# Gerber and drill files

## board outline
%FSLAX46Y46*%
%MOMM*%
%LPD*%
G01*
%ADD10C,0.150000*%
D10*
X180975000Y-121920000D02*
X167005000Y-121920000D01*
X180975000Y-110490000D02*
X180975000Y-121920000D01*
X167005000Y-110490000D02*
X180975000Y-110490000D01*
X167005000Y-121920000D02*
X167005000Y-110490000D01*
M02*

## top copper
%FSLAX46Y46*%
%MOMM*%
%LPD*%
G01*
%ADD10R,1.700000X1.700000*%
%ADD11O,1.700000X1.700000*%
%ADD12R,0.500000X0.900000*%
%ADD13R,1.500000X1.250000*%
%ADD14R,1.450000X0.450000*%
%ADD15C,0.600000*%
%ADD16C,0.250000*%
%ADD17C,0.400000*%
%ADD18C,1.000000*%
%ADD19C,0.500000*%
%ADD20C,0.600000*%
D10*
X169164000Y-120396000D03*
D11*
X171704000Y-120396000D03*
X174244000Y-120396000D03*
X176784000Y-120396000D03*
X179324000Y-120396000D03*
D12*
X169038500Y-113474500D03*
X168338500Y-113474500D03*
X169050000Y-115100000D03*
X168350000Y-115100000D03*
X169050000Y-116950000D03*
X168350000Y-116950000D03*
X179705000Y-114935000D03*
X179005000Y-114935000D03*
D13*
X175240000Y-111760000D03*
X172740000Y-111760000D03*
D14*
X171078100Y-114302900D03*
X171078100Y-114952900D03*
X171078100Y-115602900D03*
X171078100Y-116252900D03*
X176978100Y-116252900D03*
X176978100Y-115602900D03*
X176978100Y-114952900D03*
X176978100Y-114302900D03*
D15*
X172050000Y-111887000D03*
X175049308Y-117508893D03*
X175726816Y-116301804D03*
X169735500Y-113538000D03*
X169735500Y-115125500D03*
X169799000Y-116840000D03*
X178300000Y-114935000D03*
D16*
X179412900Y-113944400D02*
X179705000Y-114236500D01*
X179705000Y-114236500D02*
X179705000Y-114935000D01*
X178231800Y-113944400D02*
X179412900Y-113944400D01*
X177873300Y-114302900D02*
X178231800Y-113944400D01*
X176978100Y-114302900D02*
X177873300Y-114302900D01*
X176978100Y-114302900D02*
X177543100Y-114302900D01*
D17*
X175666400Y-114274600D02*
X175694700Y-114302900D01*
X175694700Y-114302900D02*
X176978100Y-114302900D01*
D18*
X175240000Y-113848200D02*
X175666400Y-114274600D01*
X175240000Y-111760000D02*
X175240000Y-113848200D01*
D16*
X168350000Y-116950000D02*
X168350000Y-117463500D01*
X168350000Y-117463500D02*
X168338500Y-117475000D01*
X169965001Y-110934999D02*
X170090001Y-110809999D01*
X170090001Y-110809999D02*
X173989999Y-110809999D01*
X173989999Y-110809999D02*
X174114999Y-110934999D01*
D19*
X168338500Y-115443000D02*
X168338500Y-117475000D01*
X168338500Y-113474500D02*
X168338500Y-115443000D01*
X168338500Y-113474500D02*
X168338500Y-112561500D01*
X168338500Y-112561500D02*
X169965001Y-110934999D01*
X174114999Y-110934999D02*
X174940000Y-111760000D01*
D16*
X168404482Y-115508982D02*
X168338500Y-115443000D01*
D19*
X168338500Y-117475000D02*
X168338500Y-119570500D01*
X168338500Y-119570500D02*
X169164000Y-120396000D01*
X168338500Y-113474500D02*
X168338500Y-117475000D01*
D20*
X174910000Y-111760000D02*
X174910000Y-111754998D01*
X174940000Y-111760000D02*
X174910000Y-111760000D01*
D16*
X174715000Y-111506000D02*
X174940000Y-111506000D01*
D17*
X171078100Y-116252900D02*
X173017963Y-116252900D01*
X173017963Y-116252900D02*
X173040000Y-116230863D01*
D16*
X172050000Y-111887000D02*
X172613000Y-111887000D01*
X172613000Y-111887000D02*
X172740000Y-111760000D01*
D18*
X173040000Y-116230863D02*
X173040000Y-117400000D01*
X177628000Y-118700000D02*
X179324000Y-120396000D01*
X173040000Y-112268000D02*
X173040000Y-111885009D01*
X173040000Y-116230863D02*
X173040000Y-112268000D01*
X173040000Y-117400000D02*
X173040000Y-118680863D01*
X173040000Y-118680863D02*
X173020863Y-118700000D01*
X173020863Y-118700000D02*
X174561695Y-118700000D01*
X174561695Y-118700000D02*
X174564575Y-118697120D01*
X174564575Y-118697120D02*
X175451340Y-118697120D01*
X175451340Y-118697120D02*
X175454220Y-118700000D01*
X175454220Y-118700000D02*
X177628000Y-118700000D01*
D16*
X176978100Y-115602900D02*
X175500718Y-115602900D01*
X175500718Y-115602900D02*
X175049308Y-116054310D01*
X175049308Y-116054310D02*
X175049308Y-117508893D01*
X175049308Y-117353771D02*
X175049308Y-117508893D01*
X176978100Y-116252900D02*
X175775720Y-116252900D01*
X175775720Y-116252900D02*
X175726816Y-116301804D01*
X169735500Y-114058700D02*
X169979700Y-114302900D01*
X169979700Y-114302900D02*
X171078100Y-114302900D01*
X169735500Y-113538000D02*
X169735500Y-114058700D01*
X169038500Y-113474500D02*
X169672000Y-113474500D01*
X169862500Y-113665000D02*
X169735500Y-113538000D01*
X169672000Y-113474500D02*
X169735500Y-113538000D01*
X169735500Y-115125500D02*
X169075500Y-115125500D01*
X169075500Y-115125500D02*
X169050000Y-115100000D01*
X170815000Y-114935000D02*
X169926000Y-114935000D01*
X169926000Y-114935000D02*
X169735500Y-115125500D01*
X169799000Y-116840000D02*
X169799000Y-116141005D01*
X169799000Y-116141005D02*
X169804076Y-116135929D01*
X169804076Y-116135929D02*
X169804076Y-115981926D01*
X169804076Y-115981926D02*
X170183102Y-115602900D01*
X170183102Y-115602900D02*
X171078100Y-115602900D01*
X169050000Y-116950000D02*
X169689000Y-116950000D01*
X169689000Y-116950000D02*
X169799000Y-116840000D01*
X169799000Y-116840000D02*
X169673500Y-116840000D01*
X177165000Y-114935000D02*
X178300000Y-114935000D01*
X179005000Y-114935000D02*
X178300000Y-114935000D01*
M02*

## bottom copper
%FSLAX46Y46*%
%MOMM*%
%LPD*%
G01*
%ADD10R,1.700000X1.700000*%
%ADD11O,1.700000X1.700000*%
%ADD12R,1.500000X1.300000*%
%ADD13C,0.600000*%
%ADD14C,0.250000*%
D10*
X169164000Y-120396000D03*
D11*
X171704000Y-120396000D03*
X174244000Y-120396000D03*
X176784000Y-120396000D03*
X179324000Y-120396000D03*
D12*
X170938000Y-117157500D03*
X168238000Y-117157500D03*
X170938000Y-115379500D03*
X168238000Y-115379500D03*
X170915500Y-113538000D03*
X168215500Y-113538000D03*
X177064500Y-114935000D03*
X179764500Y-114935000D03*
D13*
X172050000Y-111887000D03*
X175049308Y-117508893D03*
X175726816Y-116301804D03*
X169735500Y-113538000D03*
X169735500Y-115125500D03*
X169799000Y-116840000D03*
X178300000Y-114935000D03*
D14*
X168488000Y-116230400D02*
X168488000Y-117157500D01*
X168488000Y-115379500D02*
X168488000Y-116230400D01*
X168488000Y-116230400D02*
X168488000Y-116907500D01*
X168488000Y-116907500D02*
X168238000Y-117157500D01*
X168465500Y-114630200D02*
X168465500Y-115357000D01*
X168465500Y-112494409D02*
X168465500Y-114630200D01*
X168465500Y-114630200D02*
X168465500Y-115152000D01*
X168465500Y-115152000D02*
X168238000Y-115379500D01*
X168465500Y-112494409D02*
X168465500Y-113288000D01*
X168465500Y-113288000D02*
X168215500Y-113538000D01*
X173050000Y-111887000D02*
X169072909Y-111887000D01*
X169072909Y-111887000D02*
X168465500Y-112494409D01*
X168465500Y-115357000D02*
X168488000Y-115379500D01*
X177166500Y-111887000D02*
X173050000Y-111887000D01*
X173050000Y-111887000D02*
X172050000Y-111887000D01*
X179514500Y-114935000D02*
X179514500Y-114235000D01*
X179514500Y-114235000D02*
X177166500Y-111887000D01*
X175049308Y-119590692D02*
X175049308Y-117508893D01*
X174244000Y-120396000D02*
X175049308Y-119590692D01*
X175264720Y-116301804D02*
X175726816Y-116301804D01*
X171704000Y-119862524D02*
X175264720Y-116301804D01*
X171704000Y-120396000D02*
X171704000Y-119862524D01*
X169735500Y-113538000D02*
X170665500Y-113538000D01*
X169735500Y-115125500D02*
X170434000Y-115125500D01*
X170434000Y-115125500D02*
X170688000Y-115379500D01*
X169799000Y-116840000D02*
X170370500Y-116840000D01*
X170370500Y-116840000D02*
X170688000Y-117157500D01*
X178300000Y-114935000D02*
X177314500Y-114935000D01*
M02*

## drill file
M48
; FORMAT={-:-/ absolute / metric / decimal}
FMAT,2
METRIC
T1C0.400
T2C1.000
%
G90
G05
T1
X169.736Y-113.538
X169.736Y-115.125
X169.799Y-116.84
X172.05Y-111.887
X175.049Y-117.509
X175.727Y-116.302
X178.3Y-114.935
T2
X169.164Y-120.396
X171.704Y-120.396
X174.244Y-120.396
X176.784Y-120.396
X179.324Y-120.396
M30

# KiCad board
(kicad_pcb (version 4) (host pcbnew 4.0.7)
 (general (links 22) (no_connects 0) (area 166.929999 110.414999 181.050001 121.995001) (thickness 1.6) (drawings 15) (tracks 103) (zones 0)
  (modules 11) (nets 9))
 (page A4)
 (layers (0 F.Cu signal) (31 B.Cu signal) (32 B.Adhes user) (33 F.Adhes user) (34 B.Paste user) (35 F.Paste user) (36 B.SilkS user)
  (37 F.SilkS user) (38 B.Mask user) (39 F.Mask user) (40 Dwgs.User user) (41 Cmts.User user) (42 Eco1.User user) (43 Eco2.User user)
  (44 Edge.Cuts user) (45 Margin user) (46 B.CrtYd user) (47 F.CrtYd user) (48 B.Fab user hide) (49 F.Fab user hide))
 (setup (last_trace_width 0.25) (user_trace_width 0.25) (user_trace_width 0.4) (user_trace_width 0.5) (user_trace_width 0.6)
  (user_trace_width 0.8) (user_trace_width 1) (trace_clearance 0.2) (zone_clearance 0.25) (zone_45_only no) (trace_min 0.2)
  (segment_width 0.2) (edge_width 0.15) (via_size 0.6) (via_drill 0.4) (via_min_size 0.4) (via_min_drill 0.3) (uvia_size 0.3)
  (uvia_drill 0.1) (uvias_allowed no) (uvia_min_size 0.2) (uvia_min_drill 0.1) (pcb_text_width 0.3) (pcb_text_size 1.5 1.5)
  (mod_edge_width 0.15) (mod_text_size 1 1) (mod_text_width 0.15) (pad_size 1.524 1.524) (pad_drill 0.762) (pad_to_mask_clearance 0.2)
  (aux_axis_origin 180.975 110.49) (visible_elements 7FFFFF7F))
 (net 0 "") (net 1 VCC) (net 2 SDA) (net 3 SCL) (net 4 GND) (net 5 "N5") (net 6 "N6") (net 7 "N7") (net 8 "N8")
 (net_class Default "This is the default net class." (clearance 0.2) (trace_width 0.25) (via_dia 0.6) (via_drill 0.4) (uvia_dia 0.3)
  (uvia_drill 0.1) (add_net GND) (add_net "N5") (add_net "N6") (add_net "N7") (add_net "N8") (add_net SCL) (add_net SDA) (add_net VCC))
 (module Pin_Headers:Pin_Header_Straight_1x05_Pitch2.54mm (layer F.Cu) (at 169.164 120.396 90)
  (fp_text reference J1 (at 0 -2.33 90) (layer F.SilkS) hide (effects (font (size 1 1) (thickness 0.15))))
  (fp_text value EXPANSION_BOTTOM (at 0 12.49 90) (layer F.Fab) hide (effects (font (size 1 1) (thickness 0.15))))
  (pad 1 thru_hole rect (at 0 0 90) (size 1.7 1.7) (drill 1) (layers *.Cu *.Mask) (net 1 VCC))
  (pad 2 thru_hole oval (at 0 2.54 90) (size 1.7 1.7) (drill 1) (layers *.Cu *.Mask) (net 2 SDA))
  (pad 3 thru_hole oval (at 0 5.08 90) (size 1.7 1.7) (drill 1) (layers *.Cu *.Mask) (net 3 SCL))
  (pad 4 thru_hole oval (at 0 7.62 90) (size 1.7 1.7) (drill 1) (layers *.Cu *.Mask))
  (pad 5 thru_hole oval (at 0 10.16 90) (size 1.7 1.7) (drill 1) (layers *.Cu *.Mask) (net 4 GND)))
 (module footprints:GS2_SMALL (layer F.Cu) (at 168.3385 113.4745 270)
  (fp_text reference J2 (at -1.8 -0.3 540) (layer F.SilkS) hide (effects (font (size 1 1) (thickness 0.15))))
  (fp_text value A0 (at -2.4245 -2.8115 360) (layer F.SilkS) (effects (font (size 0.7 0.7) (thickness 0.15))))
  (pad 1 smd rect (at 0 -0.7 270) (size 0.9 0.5) (layers F.Cu F.Paste F.Mask) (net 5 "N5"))
  (pad 2 smd rect (at 0 0 270) (size 0.9 0.5) (layers F.Cu F.Paste F.Mask) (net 1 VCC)))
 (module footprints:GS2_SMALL (layer F.Cu) (at 168.35 115.1 270)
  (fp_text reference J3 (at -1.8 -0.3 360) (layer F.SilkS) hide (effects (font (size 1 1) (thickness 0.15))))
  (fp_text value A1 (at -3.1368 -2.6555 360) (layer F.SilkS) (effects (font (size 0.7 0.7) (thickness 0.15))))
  (pad 1 smd rect (at 0 -0.7 270) (size 0.9 0.5) (layers F.Cu F.Paste F.Mask) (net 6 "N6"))
  (pad 2 smd rect (at 0 0 270) (size 0.9 0.5) (layers F.Cu F.Paste F.Mask) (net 1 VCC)))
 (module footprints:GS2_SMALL (layer F.Cu) (at 168.35 116.95 270)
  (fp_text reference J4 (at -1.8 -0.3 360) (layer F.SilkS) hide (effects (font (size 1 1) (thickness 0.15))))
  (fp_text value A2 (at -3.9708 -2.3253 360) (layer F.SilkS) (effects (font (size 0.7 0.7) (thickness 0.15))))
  (pad 1 smd rect (at 0 -0.7 270) (size 0.9 0.5) (layers F.Cu F.Paste F.Mask) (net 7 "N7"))
  (pad 2 smd rect (at 0 0 270) (size 0.9 0.5) (layers F.Cu F.Paste F.Mask) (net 1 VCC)))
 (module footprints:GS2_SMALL (layer F.Cu) (at 179.005 114.935 270)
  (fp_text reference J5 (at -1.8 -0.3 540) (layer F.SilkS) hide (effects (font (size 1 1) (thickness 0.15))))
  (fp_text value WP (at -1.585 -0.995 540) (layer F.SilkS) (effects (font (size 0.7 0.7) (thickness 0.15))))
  (pad 1 smd rect (at 0 -0.7 270) (size 0.9 0.5) (layers F.Cu F.Paste F.Mask) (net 1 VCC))
  (pad 2 smd rect (at 0 0 270) (size 0.9 0.5) (layers F.Cu F.Paste F.Mask) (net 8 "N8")))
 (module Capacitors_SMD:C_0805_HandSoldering (layer F.Cu) (at 173.99 111.76 180)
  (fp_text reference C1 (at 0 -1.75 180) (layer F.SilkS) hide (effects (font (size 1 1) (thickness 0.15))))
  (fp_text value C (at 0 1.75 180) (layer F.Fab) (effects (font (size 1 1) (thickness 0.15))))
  (pad 1 smd rect (at -1.25 0 180) (size 1.5 1.25) (layers F.Cu F.Paste F.Mask) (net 1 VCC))
  (pad 2 smd rect (at 1.25 0 180) (size 1.5 1.25) (layers F.Cu F.Paste F.Mask) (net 4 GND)))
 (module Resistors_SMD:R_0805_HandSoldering (layer B.Cu) (at 169.588 117.1575 180)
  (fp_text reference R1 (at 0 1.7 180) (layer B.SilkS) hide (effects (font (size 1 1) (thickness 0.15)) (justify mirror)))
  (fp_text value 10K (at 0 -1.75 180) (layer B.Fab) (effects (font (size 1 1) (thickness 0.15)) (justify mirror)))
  (pad 1 smd rect (at -1.35 0 180) (size 1.5 1.3) (layers B.Cu B.Paste B.Mask) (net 7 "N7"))
  (pad 2 smd rect (at 1.35 0 180) (size 1.5 1.3) (layers B.Cu B.Paste B.Mask) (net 4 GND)))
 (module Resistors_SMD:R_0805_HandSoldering (layer B.Cu) (at 169.588 115.3795 180)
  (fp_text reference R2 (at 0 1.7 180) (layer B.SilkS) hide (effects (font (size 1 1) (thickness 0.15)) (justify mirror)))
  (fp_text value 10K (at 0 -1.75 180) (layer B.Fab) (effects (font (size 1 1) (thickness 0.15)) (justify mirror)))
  (pad 1 smd rect (at -1.35 0 180) (size 1.5 1.3) (layers B.Cu B.Paste B.Mask) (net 6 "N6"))
  (pad 2 smd rect (at 1.35 0 180) (size 1.5 1.3) (layers B.Cu B.Paste B.Mask) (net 4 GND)))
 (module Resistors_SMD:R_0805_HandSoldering (layer B.Cu) (at 169.5655 113.538 180)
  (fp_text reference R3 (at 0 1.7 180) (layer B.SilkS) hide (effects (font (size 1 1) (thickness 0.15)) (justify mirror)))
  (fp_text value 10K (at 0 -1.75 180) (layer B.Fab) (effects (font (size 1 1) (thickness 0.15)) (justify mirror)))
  (pad 1 smd rect (at -1.35 0 180) (size 1.5 1.3) (layers B.Cu B.Paste B.Mask) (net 5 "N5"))
  (pad 2 smd rect (at 1.35 0 180) (size 1.5 1.3) (layers B.Cu B.Paste B.Mask) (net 4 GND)))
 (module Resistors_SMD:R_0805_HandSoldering (layer B.Cu) (at 178.4145 114.935)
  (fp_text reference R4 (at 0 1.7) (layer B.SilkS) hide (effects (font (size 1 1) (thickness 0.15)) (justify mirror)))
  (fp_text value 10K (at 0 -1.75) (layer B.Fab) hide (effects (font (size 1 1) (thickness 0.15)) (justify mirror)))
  (pad 1 smd rect (at -1.35 0) (size 1.5 1.3) (layers B.Cu B.Paste B.Mask) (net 8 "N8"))
  (pad 2 smd rect (at 1.35 0) (size 1.5 1.3) (layers B.Cu B.Paste B.Mask) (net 4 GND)))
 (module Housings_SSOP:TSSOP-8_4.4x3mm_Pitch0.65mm (layer F.Cu) (at 174.0281 115.2779)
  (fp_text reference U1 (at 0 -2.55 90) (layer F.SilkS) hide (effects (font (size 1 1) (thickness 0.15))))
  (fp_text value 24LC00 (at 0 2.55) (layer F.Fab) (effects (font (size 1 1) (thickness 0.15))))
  (pad 1 smd rect (at -2.95 -0.975) (size 1.45 0.45) (layers F.Cu F.Paste F.Mask) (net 5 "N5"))
  (pad 2 smd rect (at -2.95 -0.325) (size 1.45 0.45) (layers F.Cu F.Paste F.Mask) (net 6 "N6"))
  (pad 3 smd rect (at -2.95 0.325) (size 1.45 0.45) (layers F.Cu F.Paste F.Mask) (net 7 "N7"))
  (pad 4 smd rect (at -2.95 0.975) (size 1.45 0.45) (layers F.Cu F.Paste F.Mask) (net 4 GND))
  (pad 5 smd rect (at 2.95 0.975) (size 1.45 0.45) (layers F.Cu F.Paste F.Mask) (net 2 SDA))
  (pad 6 smd rect (at 2.95 0.325) (size 1.45 0.45) (layers F.Cu F.Paste F.Mask) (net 3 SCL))
  (pad 7 smd rect (at 2.95 -0.325) (size 1.45 0.45) (layers F.Cu F.Paste F.Mask) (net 8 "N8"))
  (pad 8 smd rect (at 2.95 -0.975) (size 1.45 0.45) (layers F.Cu F.Paste F.Mask) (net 1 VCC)))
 (gr_line (start 180.975 121.92) (end 167.005 121.92) (layer Edge.Cuts) (width 0.15))
 (gr_line (start 180.975 110.49) (end 180.975 121.92) (layer Edge.Cuts) (width 0.15))
 (gr_line (start 167.005 110.49) (end 180.975 110.49) (layer Edge.Cuts) (width 0.15))
 (gr_line (start 167.005 121.92) (end 167.005 110.49) (layer Edge.Cuts) (width 0.15))
 (segment (start 179.4129 113.9444) (end 179.705 114.2365) (width 0.25) (layer F.Cu) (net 1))
 (segment (start 179.705 114.2365) (end 179.705 114.935) (width 0.25) (layer F.Cu) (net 1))
 (segment (start 178.2318 113.9444) (end 179.4129 113.9444) (width 0.25) (layer F.Cu) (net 1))
 (segment (start 177.8733 114.3029) (end 178.2318 113.9444) (width 0.25) (layer F.Cu) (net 1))
 (segment (start 176.9781 114.3029) (end 177.8733 114.3029) (width 0.25) (layer F.Cu) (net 1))
 (segment (start 176.9781 114.3029) (end 177.5431 114.3029) (width 0.25) (layer F.Cu) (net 1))
 (segment (start 175.6664 114.2746) (end 175.6947 114.3029) (width 0.4) (layer F.Cu) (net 1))
 (segment (start 175.6947 114.3029) (end 176.9781 114.3029) (width 0.4) (layer F.Cu) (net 1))
 (segment (start 175.24 113.8482) (end 175.6664 114.2746) (width 1) (layer F.Cu) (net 1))
 (segment (start 175.24 111.76) (end 175.24 113.8482) (width 1) (layer F.Cu) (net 1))
 (segment (start 168.35 116.95) (end 168.35 117.4635) (width 0.25) (layer F.Cu) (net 1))
 (segment (start 168.35 117.4635) (end 168.3385 117.475) (width 0.25) (layer F.Cu) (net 1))
 (segment (start 169.965001 110.934999) (end 170.090001 110.809999) (width 0.25) (layer F.Cu) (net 1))
 (segment (start 170.090001 110.809999) (end 173.989999 110.809999) (width 0.25) (layer F.Cu) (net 1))
 (segment (start 173.989999 110.809999) (end 174.114999 110.934999) (width 0.25) (layer F.Cu) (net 1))
 (segment (start 168.3385 115.443) (end 168.3385 117.475) (width 0.5) (layer F.Cu) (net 1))
 (segment (start 168.3385 113.4745) (end 168.3385 115.443) (width 0.5) (layer F.Cu) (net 1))
 (segment (start 168.3385 113.4745) (end 168.3385 112.5615) (width 0.5) (layer F.Cu) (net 1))
 (segment (start 168.3385 112.5615) (end 169.965001 110.934999) (width 0.5) (layer F.Cu) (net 1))
 (segment (start 174.114999 110.934999) (end 174.94 111.76) (width 0.5) (layer F.Cu) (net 1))
 (segment (start 168.404482 115.508982) (end 168.3385 115.443) (width 0.25) (layer F.Cu) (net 1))
 (segment (start 168.3385 117.475) (end 168.3385 119.5705) (width 0.5) (layer F.Cu) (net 1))
 (segment (start 168.3385 119.5705) (end 169.164 120.396) (width 0.5) (layer F.Cu) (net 1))
 (segment (start 168.3385 113.4745) (end 168.3385 117.475) (width 0.5) (layer F.Cu) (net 1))
 (segment (start 174.91 111.76) (end 174.91 111.754998) (width 0.6) (layer F.Cu) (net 1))
 (segment (start 174.94 111.76) (end 174.91 111.76) (width 0.6) (layer F.Cu) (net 1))
 (segment (start 174.715 111.506) (end 174.94 111.506) (width 0.25) (layer F.Cu) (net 1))
 (segment (start 168.488 116.2304) (end 168.488 117.1575) (width 0.25) (layer B.Cu) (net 4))
 (segment (start 168.488 115.3795) (end 168.488 116.2304) (width 0.25) (layer B.Cu) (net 4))
 (segment (start 168.488 116.2304) (end 168.488 116.9075) (width 0.25) (layer B.Cu) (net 4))
 (segment (start 168.488 116.9075) (end 168.238 117.1575) (width 0.25) (layer B.Cu) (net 4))
 (segment (start 168.4655 114.6302) (end 168.4655 115.357) (width 0.25) (layer B.Cu) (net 4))
 (segment (start 168.4655 112.494409) (end 168.4655 114.6302) (width 0.25) (layer B.Cu) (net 4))
 (segment (start 168.4655 114.6302) (end 168.4655 115.152) (width 0.25) (layer B.Cu) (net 4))
 (segment (start 168.4655 115.152) (end 168.238 115.3795) (width 0.25) (layer B.Cu) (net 4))
 (segment (start 168.4655 112.494409) (end 168.4655 113.288) (width 0.25) (layer B.Cu) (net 4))
 (segment (start 168.4655 113.288) (end 168.2155 113.538) (width 0.25) (layer B.Cu) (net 4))
 (segment (start 173.05 111.887) (end 169.072909 111.887) (width 0.25) (layer B.Cu) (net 4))
 (segment (start 169.072909 111.887) (end 168.4655 112.494409) (width 0.25) (layer B.Cu) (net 4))
 (segment (start 168.4655 115.357) (end 168.488 115.3795) (width 0.25) (layer B.Cu) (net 4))
 (segment (start 171.0781 116.2529) (end 173.017963 116.2529) (width 0.4) (layer F.Cu) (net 4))
 (segment (start 173.017963 116.2529) (end 173.04 116.230863) (width 0.4) (layer F.Cu) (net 4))
 (segment (start 172.05 111.887) (end 172.613 111.887) (width 0.25) (layer F.Cu) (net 4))
 (segment (start 172.613 111.887) (end 172.74 111.76) (width 0.25) (layer F.Cu) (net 4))
 (segment (start 173.04 116.230863) (end 173.04 117.4) (width 1) (layer F.Cu) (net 4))
 (segment (start 177.628 118.7) (end 179.324 120.396) (width 1) (layer F.Cu) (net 4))
 (segment (start 177.1665 111.887) (end 173.05 111.887) (width 0.25) (layer B.Cu) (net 4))
 (segment (start 173.05 111.887) (end 172.05 111.887) (width 0.25) (layer B.Cu) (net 4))
 (via (at 172.05 111.887) (size 0.6) (drill 0.4) (layers F.Cu B.Cu) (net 4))
 (segment (start 173.04 112.268) (end 173.04 111.885009) (width 1) (layer F.Cu) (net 4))
 (segment (start 173.04 116.230863) (end 173.04 112.268) (width 1) (layer F.Cu) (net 4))
 (segment (start 179.5145 114.935) (end 179.5145 114.235) (width 0.25) (layer B.Cu) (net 4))
 (segment (start 179.5145 114.235) (end 177.1665 111.887) (width 0.25) (layer B.Cu) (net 4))
 (segment (start 173.04 117.4) (end 173.04 118.680863) (width 1) (layer F.Cu) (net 4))
 (segment (start 173.04 118.680863) (end 173.020863 118.7) (width 1) (layer F.Cu) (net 4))
 (segment (start 173.020863 118.7) (end 174.561695 118.7) (width 1) (layer F.Cu) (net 4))
 (segment (start 174.561695 118.7) (end 174.564575 118.69712) (width 1) (layer F.Cu) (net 4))
 (segment (start 174.564575 118.69712) (end 175.45134 118.69712) (width 1) (layer F.Cu) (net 4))
 (segment (start 175.45134 118.69712) (end 175.45422 118.7) (width 1) (layer F.Cu) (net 4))
 (segment (start 175.45422 118.7) (end 177.628 118.7) (width 1) (layer F.Cu) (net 4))
 (segment (start 176.9781 115.6029) (end 175.500718 115.6029) (width 0.25) (layer F.Cu) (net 3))
 (segment (start 175.500718 115.6029) (end 175.049308 116.05431) (width 0.25) (layer F.Cu) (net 3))
 (segment (start 175.049308 116.05431) (end 175.049308 117.508893) (width 0.25) (layer F.Cu) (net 3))
 (segment (start 175.049308 117.353771) (end 175.049308 117.508893) (width 0.25) (layer F.Cu) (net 3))
 (segment (start 175.049308 119.590692) (end 175.049308 117.508893) (width 0.25) (layer B.Cu) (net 3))
 (via (at 175.049308 117.508893) (size 0.6) (drill 0.4) (layers F.Cu B.Cu) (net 3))
 (segment (start 174.244 120.396) (end 175.049308 119.590692) (width 0.25) (layer B.Cu) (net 3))
 (segment (start 176.9781 116.2529) (end 175.77572 116.2529) (width 0.25) (layer F.Cu) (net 2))
 (segment (start 175.77572 116.2529) (end 175.726816 116.301804) (width 0.25) (layer F.Cu) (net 2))
 (segment (start 175.26472 116.301804) (end 175.726816 116.301804) (width 0.25) (layer B.Cu) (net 2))
 (segment (start 171.704 119.862524) (end 175.26472 116.301804) (width 0.25) (layer B.Cu) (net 2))
 (segment (start 171.704 120.396) (end 171.704 119.862524) (width 0.25) (layer B.Cu) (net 2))
 (via (at 175.726816 116.301804) (size 0.6) (drill 0.4) (layers F.Cu B.Cu) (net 2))
 (segment (start 169.7355 114.0587) (end 169.9797 114.3029) (width 0.25) (layer F.Cu) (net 5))
 (segment (start 169.9797 114.3029) (end 171.0781 114.3029) (width 0.25) (layer F.Cu) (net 5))
 (segment (start 169.7355 113.538) (end 169.7355 114.0587) (width 0.25) (layer F.Cu) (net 5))
 (segment (start 169.0385 113.4745) (end 169.672 113.4745) (width 0.25) (layer F.Cu) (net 5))
 (segment (start 169.8625 113.665) (end 169.7355 113.538) (width 0.25) (layer F.Cu) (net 5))
 (segment (start 169.7355 113.538) (end 170.6655 113.538) (width 0.25) (layer B.Cu) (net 5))
 (segment (start 169.672 113.4745) (end 169.7355 113.538) (width 0.25) (layer F.Cu) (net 5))
 (via (at 169.7355 113.538) (size 0.6) (drill 0.4) (layers F.Cu B.Cu) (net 5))
 (segment (start 169.7355 115.1255) (end 169.0755 115.1255) (width 0.25) (layer F.Cu) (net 6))
 (segment (start 169.0755 115.1255) (end 169.05 115.1) (width 0.25) (layer F.Cu) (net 6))
 (segment (start 169.7355 115.1255) (end 170.434 115.1255) (width 0.25) (layer B.Cu) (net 6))
 (segment (start 170.434 115.1255) (end 170.688 115.3795) (width 0.25) (layer B.Cu) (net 6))
 (segment (start 170.815 114.935) (end 169.926 114.935) (width 0.25) (layer F.Cu) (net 6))
 (segment (start 169.926 114.935) (end 169.7355 115.1255) (width 0.25) (layer F.Cu) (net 6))
 (via (at 169.7355 115.1255) (size 0.6) (drill 0.4) (layers F.Cu B.Cu) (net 6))
 (segment (start 169.799 116.84) (end 169.799 116.141005) (width 0.25) (layer F.Cu) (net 7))
 (segment (start 169.799 116.141005) (end 169.804076 116.135929) (width 0.25) (layer F.Cu) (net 7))
 (segment (start 169.804076 116.135929) (end 169.804076 115.981926) (width 0.25) (layer F.Cu) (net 7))
 (segment (start 169.804076 115.981926) (end 170.183102 115.6029) (width 0.25) (layer F.Cu) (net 7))
 (segment (start 170.183102 115.6029) (end 171.0781 115.6029) (width 0.25) (layer F.Cu) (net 7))
 (segment (start 169.05 116.95) (end 169.689 116.95) (width 0.25) (layer F.Cu) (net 7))
 (segment (start 169.689 116.95) (end 169.799 116.84) (width 0.25) (layer F.Cu) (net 7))
 (segment (start 169.799 116.84) (end 169.6735 116.84) (width 0.25) (layer F.Cu) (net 7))
 (segment (start 169.799 116.84) (end 170.3705 116.84) (width 0.25) (layer B.Cu) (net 7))
 (segment (start 170.3705 116.84) (end 170.688 117.1575) (width 0.25) (layer B.Cu) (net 7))
 (via (at 169.799 116.84) (size 0.6) (drill 0.4) (layers F.Cu B.Cu) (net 7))
 (segment (start 178.3 114.935) (end 177.3145 114.935) (width 0.25) (layer B.Cu) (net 8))
 (segment (start 177.165 114.935) (end 178.3 114.935) (width 0.25) (layer F.Cu) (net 8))
 (segment (start 179.005 114.935) (end 178.3 114.935) (width 0.25) (layer F.Cu) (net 8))
 (via (at 178.3 114.935) (size 0.6) (drill 0.4) (layers F.Cu B.Cu) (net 8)))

